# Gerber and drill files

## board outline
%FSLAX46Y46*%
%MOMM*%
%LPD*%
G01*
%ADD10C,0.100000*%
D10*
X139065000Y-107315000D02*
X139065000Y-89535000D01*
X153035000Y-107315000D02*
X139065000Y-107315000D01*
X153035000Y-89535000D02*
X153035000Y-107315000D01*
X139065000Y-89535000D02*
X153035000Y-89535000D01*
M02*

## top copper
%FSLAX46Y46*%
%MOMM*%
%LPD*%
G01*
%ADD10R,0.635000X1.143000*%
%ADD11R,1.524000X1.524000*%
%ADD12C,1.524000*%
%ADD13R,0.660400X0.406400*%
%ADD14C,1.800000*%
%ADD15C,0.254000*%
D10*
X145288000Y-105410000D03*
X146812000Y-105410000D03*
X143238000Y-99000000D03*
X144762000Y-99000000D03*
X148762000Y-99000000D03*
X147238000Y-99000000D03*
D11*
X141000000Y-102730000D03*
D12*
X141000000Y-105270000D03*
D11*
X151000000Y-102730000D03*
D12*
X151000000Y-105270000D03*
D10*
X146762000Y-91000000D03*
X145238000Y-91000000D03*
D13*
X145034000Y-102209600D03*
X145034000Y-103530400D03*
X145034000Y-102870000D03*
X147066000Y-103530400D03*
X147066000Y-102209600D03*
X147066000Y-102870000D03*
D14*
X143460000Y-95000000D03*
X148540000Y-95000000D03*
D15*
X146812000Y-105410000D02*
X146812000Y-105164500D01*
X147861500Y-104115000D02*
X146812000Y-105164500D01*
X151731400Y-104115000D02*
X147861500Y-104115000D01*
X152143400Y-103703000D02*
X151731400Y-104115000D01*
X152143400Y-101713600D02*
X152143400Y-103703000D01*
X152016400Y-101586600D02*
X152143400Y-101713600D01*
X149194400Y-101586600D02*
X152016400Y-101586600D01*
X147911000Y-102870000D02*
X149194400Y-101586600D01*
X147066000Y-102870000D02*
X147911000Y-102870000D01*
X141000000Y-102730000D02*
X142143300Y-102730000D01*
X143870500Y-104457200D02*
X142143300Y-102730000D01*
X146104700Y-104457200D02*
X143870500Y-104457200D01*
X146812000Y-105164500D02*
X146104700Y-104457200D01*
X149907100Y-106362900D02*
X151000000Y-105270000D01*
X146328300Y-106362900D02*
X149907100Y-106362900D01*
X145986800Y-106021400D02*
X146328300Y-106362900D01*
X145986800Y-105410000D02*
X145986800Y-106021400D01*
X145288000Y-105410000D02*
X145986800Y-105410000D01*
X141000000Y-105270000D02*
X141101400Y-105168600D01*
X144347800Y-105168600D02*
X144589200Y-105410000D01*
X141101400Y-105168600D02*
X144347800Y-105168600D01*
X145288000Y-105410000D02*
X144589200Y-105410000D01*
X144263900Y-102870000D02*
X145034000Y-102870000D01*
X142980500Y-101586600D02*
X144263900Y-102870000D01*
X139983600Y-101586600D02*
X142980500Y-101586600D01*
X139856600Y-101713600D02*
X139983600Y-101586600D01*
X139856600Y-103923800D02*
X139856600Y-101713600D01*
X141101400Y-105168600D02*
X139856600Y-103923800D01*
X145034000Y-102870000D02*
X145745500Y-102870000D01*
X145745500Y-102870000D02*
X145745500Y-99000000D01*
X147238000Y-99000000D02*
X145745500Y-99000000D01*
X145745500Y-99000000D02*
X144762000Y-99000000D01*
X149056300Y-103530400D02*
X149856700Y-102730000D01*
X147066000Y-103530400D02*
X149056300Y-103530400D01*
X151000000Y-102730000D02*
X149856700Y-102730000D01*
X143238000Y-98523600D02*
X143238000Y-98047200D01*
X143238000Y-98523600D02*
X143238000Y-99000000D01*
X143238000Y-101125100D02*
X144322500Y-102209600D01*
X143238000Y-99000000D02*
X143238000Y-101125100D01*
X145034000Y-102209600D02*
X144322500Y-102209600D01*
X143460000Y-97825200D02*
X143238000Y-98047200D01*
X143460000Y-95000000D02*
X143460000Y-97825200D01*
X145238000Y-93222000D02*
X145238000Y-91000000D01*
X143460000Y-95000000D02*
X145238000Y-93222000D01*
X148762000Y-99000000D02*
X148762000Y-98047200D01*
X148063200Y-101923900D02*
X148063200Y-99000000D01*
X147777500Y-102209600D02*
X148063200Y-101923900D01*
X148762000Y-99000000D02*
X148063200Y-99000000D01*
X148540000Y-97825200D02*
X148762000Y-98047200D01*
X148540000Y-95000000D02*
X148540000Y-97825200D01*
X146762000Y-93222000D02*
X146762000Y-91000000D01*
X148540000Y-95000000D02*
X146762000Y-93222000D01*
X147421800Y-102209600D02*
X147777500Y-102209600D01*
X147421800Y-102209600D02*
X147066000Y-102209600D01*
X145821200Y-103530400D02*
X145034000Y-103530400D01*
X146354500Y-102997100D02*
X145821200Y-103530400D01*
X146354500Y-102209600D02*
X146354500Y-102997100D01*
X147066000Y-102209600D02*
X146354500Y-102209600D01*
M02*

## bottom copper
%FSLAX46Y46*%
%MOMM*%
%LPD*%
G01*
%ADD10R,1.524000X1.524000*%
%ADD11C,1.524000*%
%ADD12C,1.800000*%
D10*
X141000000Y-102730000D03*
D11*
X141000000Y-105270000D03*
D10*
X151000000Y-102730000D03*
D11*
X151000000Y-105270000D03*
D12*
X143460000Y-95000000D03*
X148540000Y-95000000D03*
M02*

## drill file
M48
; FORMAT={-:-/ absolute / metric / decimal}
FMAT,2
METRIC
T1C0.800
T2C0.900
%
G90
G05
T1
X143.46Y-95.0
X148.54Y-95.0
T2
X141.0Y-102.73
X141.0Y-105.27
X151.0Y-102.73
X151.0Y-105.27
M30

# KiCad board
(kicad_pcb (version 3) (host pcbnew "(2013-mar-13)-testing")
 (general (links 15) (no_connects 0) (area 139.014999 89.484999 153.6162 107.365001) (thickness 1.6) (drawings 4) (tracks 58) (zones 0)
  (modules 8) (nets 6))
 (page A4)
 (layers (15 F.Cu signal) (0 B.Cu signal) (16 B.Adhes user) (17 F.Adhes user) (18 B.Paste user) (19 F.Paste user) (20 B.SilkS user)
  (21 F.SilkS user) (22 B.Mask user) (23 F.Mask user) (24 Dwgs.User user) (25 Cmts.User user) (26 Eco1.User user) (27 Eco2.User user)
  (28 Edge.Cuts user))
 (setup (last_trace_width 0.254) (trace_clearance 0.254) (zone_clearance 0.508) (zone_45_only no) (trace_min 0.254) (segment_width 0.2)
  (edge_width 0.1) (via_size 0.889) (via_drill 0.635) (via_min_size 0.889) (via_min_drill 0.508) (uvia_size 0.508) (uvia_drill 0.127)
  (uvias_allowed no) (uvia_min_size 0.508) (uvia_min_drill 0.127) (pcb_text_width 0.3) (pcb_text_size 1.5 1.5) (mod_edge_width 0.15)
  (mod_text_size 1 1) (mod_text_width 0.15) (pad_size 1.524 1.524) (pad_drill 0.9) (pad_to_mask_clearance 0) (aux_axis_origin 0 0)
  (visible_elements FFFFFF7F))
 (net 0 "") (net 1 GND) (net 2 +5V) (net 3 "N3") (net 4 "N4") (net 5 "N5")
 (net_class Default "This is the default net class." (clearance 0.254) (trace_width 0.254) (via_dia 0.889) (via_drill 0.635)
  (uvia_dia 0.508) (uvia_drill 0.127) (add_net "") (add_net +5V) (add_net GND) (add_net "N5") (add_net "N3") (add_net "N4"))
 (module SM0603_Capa (layer F.Cu) (at 146.05 105.41)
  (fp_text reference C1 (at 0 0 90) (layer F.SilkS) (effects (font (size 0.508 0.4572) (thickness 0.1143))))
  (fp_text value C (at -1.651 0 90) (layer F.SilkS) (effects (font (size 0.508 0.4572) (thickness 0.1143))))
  (pad 1 smd rect (at -0.762 0) (size 0.635 1.143) (layers F.Cu F.Paste F.Mask) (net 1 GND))
  (pad 2 smd rect (at 0.762 0) (size 0.635 1.143) (layers F.Cu F.Paste F.Mask) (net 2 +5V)))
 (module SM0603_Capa (layer F.Cu) (at 144 99)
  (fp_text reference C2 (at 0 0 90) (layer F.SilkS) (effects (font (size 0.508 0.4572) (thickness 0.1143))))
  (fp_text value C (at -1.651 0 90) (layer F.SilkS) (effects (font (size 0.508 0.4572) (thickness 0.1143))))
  (pad 1 smd rect (at -0.762 0) (size 0.635 1.143) (layers F.Cu F.Paste F.Mask) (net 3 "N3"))
  (pad 2 smd rect (at 0.762 0) (size 0.635 1.143) (layers F.Cu F.Paste F.Mask) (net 1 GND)))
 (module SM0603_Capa (layer F.Cu) (at 148 99 180)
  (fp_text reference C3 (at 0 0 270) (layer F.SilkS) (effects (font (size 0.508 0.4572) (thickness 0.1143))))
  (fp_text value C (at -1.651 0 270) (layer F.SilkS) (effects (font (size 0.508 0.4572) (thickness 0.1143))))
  (pad 1 smd rect (at -0.762 0 180) (size 0.635 1.143) (layers F.Cu F.Paste F.Mask) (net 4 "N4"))
  (pad 2 smd rect (at 0.762 0 180) (size 0.635 1.143) (layers F.Cu F.Paste F.Mask) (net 1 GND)))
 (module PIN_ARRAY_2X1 (layer F.Cu) (at 141 104 270)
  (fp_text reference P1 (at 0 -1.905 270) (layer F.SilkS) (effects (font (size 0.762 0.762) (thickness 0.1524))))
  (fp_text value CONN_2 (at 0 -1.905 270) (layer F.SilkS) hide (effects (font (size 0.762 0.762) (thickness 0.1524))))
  (pad 1 thru_hole rect (at -1.27 0 270) (size 1.524 1.524) (drill 0.9) (layers *.Cu *.Mask F.SilkS) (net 2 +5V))
  (pad 2 thru_hole circle (at 1.27 0 270) (size 1.524 1.524) (drill 0.9) (layers *.Cu *.Mask F.SilkS) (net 1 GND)))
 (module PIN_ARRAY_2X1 (layer F.Cu) (at 151 104 270)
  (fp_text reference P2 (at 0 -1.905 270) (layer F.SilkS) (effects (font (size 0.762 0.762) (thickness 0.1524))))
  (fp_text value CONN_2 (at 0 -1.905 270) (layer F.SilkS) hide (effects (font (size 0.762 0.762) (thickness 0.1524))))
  (pad 1 thru_hole rect (at -1.27 0 270) (size 1.524 1.524) (drill 0.9) (layers *.Cu *.Mask F.SilkS) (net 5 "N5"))
  (pad 2 thru_hole circle (at 1.27 0 270) (size 1.524 1.524) (drill 0.9) (layers *.Cu *.Mask F.SilkS) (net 1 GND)))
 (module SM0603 (layer F.Cu) (at 146 91 180)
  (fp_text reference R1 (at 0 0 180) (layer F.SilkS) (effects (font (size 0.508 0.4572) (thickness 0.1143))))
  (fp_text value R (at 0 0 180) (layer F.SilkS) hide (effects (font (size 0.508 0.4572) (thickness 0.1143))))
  (pad 1 smd rect (at -0.762 0 180) (size 0.635 1.143) (layers F.Cu F.Paste F.Mask) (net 4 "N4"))
  (pad 2 smd rect (at 0.762 0 180) (size 0.635 1.143) (layers F.Cu F.Paste F.Mask) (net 3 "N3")))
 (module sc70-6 (layer F.Cu) (at 146.05 102.87 270)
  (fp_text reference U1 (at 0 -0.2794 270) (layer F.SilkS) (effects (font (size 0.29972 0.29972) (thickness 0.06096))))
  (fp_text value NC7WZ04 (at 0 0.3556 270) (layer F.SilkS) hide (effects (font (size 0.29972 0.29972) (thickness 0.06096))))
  (pad 1 smd rect (at -0.6604 1.016 270) (size 0.4064 0.6604) (layers F.Cu F.Paste F.Mask) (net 3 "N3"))
  (pad 3 smd rect (at 0.6604 1.016 270) (size 0.4064 0.6604) (layers F.Cu F.Paste F.Mask) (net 4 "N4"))
  (pad 2 smd rect (at 0 1.016 270) (size 0.4064 0.6604) (layers F.Cu F.Paste F.Mask) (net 1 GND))
  (pad 4 smd rect (at 0.6604 -1.016 270) (size 0.4064 0.6604) (layers F.Cu F.Paste F.Mask) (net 5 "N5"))
  (pad 6 smd rect (at -0.6604 -1.016 270) (size 0.4064 0.6604) (layers F.Cu F.Paste F.Mask) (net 4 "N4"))
  (pad 5 smd rect (at 0 -1.016 270) (size 0.4064 0.6604) (layers F.Cu F.Paste F.Mask) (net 2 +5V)))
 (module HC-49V (layer F.Cu) (at 146 95) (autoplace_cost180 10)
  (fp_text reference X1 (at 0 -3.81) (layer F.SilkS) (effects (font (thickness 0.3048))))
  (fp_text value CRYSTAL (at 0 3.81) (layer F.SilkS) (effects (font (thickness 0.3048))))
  (pad 1 thru_hole circle (at -2.54 0) (size 1.8 1.8) (drill 0.8) (layers *.Cu *.Mask F.SilkS) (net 3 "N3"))
  (pad 2 thru_hole circle (at 2.54 0) (size 1.8 1.8) (drill 0.8) (layers *.Cu *.Mask F.SilkS) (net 4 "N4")))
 (gr_line (start 139.065 107.315) (end 139.065 89.535) (angle 90) (layer Edge.Cuts) (width 0.1))
 (gr_line (start 153.035 107.315) (end 139.065 107.315) (angle 90) (layer Edge.Cuts) (width 0.1))
 (gr_line (start 153.035 89.535) (end 153.035 107.315) (angle 90) (layer Edge.Cuts) (width 0.1))
 (gr_line (start 139.065 89.535) (end 153.035 89.535) (angle 90) (layer Edge.Cuts) (width 0.1))
 (segment (start 146.812 105.41) (end 146.812 105.1645) (width 0.254) (layer F.Cu) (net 2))
 (segment (start 147.8615 104.115) (end 146.812 105.1645) (width 0.254) (layer F.Cu) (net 2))
 (segment (start 151.7314 104.115) (end 147.8615 104.115) (width 0.254) (layer F.Cu) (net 2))
 (segment (start 152.1434 103.703) (end 151.7314 104.115) (width 0.254) (layer F.Cu) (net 2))
 (segment (start 152.1434 101.7136) (end 152.1434 103.703) (width 0.254) (layer F.Cu) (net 2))
 (segment (start 152.0164 101.5866) (end 152.1434 101.7136) (width 0.254) (layer F.Cu) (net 2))
 (segment (start 149.1944 101.5866) (end 152.0164 101.5866) (width 0.254) (layer F.Cu) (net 2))
 (segment (start 147.911 102.87) (end 149.1944 101.5866) (width 0.254) (layer F.Cu) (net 2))
 (segment (start 147.066 102.87) (end 147.911 102.87) (width 0.254) (layer F.Cu) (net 2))
 (segment (start 141 102.73) (end 142.1433 102.73) (width 0.254) (layer F.Cu) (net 2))
 (segment (start 143.8705 104.4572) (end 142.1433 102.73) (width 0.254) (layer F.Cu) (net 2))
 (segment (start 146.1047 104.4572) (end 143.8705 104.4572) (width 0.254) (layer F.Cu) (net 2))
 (segment (start 146.812 105.1645) (end 146.1047 104.4572) (width 0.254) (layer F.Cu) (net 2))
 (segment (start 149.9071 106.3629) (end 151 105.27) (width 0.254) (layer F.Cu) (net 1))
 (segment (start 146.3283 106.3629) (end 149.9071 106.3629) (width 0.254) (layer F.Cu) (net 1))
 (segment (start 145.9868 106.0214) (end 146.3283 106.3629) (width 0.254) (layer F.Cu) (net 1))
 (segment (start 145.9868 105.41) (end 145.9868 106.0214) (width 0.254) (layer F.Cu) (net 1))
 (segment (start 145.288 105.41) (end 145.9868 105.41) (width 0.254) (layer F.Cu) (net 1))
 (segment (start 141 105.27) (end 141.1014 105.1686) (width 0.254) (layer F.Cu) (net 1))
 (segment (start 144.3478 105.1686) (end 144.5892 105.41) (width 0.254) (layer F.Cu) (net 1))
 (segment (start 141.1014 105.1686) (end 144.3478 105.1686) (width 0.254) (layer F.Cu) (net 1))
 (segment (start 145.288 105.41) (end 144.5892 105.41) (width 0.254) (layer F.Cu) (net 1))
 (segment (start 144.2639 102.87) (end 145.034 102.87) (width 0.254) (layer F.Cu) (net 1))
 (segment (start 142.9805 101.5866) (end 144.2639 102.87) (width 0.254) (layer F.Cu) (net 1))
 (segment (start 139.9836 101.5866) (end 142.9805 101.5866) (width 0.254) (layer F.Cu) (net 1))
 (segment (start 139.8566 101.7136) (end 139.9836 101.5866) (width 0.254) (layer F.Cu) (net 1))
 (segment (start 139.8566 103.9238) (end 139.8566 101.7136) (width 0.254) (layer F.Cu) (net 1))
 (segment (start 141.1014 105.1686) (end 139.8566 103.9238) (width 0.254) (layer F.Cu) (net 1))
 (segment (start 145.034 102.87) (end 145.7455 102.87) (width 0.254) (layer F.Cu) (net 1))
 (segment (start 145.7455 102.87) (end 145.7455 99) (width 0.254) (layer F.Cu) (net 1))
 (segment (start 147.238 99) (end 145.7455 99) (width 0.254) (layer F.Cu) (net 1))
 (segment (start 145.7455 99) (end 144.762 99) (width 0.254) (layer F.Cu) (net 1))
 (segment (start 149.0563 103.5304) (end 149.8567 102.73) (width 0.254) (layer F.Cu) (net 5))
 (segment (start 147.066 103.5304) (end 149.0563 103.5304) (width 0.254) (layer F.Cu) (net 5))
 (segment (start 151 102.73) (end 149.8567 102.73) (width 0.254) (layer F.Cu) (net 5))
 (segment (start 143.238 98.5236) (end 143.238 98.0472) (width 0.254) (layer F.Cu) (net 3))
 (segment (start 143.238 98.5236) (end 143.238 99) (width 0.254) (layer F.Cu) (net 3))
 (segment (start 143.238 101.1251) (end 144.3225 102.2096) (width 0.254) (layer F.Cu) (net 3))
 (segment (start 143.238 99) (end 143.238 101.1251) (width 0.254) (layer F.Cu) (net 3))
 (segment (start 145.034 102.2096) (end 144.3225 102.2096) (width 0.254) (layer F.Cu) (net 3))
 (segment (start 143.46 97.8252) (end 143.238 98.0472) (width 0.254) (layer F.Cu) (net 3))
 (segment (start 143.46 95) (end 143.46 97.8252) (width 0.254) (layer F.Cu) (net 3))
 (segment (start 145.238 93.222) (end 145.238 91) (width 0.254) (layer F.Cu) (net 3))
 (segment (start 143.46 95) (end 145.238 93.222) (width 0.254) (layer F.Cu) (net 3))
 (segment (start 148.762 99) (end 148.762 98.0472) (width 0.254) (layer F.Cu) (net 4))
 (segment (start 148.0632 101.9239) (end 148.0632 99) (width 0.254) (layer F.Cu) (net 4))
 (segment (start 147.7775 102.2096) (end 148.0632 101.9239) (width 0.254) (layer F.Cu) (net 4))
 (segment (start 148.762 99) (end 148.0632 99) (width 0.254) (layer F.Cu) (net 4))
 (segment (start 148.54 97.8252) (end 148.762 98.0472) (width 0.254) (layer F.Cu) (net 4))
 (segment (start 148.54 95) (end 148.54 97.8252) (width 0.254) (layer F.Cu) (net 4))
 (segment (start 146.762 93.222) (end 146.762 91) (width 0.254) (layer F.Cu) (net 4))
 (segment (start 148.54 95) (end 146.762 93.222) (width 0.254) (layer F.Cu) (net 4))
 (segment (start 147.4218 102.2096) (end 147.7775 102.2096) (width 0.254) (layer F.Cu) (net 4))
 (segment (start 147.4218 102.2096) (end 147.066 102.2096) (width 0.254) (layer F.Cu) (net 4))
 (segment (start 145.8212 103.5304) (end 145.034 103.5304) (width 0.254) (layer F.Cu) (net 4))
 (segment (start 146.3545 102.9971) (end 145.8212 103.5304) (width 0.254) (layer F.Cu) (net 4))
 (segment (start 146.3545 102.2096) (end 146.3545 102.9971) (width 0.254) (layer F.Cu) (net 4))
 (segment (start 147.066 102.2096) (end 146.3545 102.2096) (width 0.254) (layer F.Cu) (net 4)))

